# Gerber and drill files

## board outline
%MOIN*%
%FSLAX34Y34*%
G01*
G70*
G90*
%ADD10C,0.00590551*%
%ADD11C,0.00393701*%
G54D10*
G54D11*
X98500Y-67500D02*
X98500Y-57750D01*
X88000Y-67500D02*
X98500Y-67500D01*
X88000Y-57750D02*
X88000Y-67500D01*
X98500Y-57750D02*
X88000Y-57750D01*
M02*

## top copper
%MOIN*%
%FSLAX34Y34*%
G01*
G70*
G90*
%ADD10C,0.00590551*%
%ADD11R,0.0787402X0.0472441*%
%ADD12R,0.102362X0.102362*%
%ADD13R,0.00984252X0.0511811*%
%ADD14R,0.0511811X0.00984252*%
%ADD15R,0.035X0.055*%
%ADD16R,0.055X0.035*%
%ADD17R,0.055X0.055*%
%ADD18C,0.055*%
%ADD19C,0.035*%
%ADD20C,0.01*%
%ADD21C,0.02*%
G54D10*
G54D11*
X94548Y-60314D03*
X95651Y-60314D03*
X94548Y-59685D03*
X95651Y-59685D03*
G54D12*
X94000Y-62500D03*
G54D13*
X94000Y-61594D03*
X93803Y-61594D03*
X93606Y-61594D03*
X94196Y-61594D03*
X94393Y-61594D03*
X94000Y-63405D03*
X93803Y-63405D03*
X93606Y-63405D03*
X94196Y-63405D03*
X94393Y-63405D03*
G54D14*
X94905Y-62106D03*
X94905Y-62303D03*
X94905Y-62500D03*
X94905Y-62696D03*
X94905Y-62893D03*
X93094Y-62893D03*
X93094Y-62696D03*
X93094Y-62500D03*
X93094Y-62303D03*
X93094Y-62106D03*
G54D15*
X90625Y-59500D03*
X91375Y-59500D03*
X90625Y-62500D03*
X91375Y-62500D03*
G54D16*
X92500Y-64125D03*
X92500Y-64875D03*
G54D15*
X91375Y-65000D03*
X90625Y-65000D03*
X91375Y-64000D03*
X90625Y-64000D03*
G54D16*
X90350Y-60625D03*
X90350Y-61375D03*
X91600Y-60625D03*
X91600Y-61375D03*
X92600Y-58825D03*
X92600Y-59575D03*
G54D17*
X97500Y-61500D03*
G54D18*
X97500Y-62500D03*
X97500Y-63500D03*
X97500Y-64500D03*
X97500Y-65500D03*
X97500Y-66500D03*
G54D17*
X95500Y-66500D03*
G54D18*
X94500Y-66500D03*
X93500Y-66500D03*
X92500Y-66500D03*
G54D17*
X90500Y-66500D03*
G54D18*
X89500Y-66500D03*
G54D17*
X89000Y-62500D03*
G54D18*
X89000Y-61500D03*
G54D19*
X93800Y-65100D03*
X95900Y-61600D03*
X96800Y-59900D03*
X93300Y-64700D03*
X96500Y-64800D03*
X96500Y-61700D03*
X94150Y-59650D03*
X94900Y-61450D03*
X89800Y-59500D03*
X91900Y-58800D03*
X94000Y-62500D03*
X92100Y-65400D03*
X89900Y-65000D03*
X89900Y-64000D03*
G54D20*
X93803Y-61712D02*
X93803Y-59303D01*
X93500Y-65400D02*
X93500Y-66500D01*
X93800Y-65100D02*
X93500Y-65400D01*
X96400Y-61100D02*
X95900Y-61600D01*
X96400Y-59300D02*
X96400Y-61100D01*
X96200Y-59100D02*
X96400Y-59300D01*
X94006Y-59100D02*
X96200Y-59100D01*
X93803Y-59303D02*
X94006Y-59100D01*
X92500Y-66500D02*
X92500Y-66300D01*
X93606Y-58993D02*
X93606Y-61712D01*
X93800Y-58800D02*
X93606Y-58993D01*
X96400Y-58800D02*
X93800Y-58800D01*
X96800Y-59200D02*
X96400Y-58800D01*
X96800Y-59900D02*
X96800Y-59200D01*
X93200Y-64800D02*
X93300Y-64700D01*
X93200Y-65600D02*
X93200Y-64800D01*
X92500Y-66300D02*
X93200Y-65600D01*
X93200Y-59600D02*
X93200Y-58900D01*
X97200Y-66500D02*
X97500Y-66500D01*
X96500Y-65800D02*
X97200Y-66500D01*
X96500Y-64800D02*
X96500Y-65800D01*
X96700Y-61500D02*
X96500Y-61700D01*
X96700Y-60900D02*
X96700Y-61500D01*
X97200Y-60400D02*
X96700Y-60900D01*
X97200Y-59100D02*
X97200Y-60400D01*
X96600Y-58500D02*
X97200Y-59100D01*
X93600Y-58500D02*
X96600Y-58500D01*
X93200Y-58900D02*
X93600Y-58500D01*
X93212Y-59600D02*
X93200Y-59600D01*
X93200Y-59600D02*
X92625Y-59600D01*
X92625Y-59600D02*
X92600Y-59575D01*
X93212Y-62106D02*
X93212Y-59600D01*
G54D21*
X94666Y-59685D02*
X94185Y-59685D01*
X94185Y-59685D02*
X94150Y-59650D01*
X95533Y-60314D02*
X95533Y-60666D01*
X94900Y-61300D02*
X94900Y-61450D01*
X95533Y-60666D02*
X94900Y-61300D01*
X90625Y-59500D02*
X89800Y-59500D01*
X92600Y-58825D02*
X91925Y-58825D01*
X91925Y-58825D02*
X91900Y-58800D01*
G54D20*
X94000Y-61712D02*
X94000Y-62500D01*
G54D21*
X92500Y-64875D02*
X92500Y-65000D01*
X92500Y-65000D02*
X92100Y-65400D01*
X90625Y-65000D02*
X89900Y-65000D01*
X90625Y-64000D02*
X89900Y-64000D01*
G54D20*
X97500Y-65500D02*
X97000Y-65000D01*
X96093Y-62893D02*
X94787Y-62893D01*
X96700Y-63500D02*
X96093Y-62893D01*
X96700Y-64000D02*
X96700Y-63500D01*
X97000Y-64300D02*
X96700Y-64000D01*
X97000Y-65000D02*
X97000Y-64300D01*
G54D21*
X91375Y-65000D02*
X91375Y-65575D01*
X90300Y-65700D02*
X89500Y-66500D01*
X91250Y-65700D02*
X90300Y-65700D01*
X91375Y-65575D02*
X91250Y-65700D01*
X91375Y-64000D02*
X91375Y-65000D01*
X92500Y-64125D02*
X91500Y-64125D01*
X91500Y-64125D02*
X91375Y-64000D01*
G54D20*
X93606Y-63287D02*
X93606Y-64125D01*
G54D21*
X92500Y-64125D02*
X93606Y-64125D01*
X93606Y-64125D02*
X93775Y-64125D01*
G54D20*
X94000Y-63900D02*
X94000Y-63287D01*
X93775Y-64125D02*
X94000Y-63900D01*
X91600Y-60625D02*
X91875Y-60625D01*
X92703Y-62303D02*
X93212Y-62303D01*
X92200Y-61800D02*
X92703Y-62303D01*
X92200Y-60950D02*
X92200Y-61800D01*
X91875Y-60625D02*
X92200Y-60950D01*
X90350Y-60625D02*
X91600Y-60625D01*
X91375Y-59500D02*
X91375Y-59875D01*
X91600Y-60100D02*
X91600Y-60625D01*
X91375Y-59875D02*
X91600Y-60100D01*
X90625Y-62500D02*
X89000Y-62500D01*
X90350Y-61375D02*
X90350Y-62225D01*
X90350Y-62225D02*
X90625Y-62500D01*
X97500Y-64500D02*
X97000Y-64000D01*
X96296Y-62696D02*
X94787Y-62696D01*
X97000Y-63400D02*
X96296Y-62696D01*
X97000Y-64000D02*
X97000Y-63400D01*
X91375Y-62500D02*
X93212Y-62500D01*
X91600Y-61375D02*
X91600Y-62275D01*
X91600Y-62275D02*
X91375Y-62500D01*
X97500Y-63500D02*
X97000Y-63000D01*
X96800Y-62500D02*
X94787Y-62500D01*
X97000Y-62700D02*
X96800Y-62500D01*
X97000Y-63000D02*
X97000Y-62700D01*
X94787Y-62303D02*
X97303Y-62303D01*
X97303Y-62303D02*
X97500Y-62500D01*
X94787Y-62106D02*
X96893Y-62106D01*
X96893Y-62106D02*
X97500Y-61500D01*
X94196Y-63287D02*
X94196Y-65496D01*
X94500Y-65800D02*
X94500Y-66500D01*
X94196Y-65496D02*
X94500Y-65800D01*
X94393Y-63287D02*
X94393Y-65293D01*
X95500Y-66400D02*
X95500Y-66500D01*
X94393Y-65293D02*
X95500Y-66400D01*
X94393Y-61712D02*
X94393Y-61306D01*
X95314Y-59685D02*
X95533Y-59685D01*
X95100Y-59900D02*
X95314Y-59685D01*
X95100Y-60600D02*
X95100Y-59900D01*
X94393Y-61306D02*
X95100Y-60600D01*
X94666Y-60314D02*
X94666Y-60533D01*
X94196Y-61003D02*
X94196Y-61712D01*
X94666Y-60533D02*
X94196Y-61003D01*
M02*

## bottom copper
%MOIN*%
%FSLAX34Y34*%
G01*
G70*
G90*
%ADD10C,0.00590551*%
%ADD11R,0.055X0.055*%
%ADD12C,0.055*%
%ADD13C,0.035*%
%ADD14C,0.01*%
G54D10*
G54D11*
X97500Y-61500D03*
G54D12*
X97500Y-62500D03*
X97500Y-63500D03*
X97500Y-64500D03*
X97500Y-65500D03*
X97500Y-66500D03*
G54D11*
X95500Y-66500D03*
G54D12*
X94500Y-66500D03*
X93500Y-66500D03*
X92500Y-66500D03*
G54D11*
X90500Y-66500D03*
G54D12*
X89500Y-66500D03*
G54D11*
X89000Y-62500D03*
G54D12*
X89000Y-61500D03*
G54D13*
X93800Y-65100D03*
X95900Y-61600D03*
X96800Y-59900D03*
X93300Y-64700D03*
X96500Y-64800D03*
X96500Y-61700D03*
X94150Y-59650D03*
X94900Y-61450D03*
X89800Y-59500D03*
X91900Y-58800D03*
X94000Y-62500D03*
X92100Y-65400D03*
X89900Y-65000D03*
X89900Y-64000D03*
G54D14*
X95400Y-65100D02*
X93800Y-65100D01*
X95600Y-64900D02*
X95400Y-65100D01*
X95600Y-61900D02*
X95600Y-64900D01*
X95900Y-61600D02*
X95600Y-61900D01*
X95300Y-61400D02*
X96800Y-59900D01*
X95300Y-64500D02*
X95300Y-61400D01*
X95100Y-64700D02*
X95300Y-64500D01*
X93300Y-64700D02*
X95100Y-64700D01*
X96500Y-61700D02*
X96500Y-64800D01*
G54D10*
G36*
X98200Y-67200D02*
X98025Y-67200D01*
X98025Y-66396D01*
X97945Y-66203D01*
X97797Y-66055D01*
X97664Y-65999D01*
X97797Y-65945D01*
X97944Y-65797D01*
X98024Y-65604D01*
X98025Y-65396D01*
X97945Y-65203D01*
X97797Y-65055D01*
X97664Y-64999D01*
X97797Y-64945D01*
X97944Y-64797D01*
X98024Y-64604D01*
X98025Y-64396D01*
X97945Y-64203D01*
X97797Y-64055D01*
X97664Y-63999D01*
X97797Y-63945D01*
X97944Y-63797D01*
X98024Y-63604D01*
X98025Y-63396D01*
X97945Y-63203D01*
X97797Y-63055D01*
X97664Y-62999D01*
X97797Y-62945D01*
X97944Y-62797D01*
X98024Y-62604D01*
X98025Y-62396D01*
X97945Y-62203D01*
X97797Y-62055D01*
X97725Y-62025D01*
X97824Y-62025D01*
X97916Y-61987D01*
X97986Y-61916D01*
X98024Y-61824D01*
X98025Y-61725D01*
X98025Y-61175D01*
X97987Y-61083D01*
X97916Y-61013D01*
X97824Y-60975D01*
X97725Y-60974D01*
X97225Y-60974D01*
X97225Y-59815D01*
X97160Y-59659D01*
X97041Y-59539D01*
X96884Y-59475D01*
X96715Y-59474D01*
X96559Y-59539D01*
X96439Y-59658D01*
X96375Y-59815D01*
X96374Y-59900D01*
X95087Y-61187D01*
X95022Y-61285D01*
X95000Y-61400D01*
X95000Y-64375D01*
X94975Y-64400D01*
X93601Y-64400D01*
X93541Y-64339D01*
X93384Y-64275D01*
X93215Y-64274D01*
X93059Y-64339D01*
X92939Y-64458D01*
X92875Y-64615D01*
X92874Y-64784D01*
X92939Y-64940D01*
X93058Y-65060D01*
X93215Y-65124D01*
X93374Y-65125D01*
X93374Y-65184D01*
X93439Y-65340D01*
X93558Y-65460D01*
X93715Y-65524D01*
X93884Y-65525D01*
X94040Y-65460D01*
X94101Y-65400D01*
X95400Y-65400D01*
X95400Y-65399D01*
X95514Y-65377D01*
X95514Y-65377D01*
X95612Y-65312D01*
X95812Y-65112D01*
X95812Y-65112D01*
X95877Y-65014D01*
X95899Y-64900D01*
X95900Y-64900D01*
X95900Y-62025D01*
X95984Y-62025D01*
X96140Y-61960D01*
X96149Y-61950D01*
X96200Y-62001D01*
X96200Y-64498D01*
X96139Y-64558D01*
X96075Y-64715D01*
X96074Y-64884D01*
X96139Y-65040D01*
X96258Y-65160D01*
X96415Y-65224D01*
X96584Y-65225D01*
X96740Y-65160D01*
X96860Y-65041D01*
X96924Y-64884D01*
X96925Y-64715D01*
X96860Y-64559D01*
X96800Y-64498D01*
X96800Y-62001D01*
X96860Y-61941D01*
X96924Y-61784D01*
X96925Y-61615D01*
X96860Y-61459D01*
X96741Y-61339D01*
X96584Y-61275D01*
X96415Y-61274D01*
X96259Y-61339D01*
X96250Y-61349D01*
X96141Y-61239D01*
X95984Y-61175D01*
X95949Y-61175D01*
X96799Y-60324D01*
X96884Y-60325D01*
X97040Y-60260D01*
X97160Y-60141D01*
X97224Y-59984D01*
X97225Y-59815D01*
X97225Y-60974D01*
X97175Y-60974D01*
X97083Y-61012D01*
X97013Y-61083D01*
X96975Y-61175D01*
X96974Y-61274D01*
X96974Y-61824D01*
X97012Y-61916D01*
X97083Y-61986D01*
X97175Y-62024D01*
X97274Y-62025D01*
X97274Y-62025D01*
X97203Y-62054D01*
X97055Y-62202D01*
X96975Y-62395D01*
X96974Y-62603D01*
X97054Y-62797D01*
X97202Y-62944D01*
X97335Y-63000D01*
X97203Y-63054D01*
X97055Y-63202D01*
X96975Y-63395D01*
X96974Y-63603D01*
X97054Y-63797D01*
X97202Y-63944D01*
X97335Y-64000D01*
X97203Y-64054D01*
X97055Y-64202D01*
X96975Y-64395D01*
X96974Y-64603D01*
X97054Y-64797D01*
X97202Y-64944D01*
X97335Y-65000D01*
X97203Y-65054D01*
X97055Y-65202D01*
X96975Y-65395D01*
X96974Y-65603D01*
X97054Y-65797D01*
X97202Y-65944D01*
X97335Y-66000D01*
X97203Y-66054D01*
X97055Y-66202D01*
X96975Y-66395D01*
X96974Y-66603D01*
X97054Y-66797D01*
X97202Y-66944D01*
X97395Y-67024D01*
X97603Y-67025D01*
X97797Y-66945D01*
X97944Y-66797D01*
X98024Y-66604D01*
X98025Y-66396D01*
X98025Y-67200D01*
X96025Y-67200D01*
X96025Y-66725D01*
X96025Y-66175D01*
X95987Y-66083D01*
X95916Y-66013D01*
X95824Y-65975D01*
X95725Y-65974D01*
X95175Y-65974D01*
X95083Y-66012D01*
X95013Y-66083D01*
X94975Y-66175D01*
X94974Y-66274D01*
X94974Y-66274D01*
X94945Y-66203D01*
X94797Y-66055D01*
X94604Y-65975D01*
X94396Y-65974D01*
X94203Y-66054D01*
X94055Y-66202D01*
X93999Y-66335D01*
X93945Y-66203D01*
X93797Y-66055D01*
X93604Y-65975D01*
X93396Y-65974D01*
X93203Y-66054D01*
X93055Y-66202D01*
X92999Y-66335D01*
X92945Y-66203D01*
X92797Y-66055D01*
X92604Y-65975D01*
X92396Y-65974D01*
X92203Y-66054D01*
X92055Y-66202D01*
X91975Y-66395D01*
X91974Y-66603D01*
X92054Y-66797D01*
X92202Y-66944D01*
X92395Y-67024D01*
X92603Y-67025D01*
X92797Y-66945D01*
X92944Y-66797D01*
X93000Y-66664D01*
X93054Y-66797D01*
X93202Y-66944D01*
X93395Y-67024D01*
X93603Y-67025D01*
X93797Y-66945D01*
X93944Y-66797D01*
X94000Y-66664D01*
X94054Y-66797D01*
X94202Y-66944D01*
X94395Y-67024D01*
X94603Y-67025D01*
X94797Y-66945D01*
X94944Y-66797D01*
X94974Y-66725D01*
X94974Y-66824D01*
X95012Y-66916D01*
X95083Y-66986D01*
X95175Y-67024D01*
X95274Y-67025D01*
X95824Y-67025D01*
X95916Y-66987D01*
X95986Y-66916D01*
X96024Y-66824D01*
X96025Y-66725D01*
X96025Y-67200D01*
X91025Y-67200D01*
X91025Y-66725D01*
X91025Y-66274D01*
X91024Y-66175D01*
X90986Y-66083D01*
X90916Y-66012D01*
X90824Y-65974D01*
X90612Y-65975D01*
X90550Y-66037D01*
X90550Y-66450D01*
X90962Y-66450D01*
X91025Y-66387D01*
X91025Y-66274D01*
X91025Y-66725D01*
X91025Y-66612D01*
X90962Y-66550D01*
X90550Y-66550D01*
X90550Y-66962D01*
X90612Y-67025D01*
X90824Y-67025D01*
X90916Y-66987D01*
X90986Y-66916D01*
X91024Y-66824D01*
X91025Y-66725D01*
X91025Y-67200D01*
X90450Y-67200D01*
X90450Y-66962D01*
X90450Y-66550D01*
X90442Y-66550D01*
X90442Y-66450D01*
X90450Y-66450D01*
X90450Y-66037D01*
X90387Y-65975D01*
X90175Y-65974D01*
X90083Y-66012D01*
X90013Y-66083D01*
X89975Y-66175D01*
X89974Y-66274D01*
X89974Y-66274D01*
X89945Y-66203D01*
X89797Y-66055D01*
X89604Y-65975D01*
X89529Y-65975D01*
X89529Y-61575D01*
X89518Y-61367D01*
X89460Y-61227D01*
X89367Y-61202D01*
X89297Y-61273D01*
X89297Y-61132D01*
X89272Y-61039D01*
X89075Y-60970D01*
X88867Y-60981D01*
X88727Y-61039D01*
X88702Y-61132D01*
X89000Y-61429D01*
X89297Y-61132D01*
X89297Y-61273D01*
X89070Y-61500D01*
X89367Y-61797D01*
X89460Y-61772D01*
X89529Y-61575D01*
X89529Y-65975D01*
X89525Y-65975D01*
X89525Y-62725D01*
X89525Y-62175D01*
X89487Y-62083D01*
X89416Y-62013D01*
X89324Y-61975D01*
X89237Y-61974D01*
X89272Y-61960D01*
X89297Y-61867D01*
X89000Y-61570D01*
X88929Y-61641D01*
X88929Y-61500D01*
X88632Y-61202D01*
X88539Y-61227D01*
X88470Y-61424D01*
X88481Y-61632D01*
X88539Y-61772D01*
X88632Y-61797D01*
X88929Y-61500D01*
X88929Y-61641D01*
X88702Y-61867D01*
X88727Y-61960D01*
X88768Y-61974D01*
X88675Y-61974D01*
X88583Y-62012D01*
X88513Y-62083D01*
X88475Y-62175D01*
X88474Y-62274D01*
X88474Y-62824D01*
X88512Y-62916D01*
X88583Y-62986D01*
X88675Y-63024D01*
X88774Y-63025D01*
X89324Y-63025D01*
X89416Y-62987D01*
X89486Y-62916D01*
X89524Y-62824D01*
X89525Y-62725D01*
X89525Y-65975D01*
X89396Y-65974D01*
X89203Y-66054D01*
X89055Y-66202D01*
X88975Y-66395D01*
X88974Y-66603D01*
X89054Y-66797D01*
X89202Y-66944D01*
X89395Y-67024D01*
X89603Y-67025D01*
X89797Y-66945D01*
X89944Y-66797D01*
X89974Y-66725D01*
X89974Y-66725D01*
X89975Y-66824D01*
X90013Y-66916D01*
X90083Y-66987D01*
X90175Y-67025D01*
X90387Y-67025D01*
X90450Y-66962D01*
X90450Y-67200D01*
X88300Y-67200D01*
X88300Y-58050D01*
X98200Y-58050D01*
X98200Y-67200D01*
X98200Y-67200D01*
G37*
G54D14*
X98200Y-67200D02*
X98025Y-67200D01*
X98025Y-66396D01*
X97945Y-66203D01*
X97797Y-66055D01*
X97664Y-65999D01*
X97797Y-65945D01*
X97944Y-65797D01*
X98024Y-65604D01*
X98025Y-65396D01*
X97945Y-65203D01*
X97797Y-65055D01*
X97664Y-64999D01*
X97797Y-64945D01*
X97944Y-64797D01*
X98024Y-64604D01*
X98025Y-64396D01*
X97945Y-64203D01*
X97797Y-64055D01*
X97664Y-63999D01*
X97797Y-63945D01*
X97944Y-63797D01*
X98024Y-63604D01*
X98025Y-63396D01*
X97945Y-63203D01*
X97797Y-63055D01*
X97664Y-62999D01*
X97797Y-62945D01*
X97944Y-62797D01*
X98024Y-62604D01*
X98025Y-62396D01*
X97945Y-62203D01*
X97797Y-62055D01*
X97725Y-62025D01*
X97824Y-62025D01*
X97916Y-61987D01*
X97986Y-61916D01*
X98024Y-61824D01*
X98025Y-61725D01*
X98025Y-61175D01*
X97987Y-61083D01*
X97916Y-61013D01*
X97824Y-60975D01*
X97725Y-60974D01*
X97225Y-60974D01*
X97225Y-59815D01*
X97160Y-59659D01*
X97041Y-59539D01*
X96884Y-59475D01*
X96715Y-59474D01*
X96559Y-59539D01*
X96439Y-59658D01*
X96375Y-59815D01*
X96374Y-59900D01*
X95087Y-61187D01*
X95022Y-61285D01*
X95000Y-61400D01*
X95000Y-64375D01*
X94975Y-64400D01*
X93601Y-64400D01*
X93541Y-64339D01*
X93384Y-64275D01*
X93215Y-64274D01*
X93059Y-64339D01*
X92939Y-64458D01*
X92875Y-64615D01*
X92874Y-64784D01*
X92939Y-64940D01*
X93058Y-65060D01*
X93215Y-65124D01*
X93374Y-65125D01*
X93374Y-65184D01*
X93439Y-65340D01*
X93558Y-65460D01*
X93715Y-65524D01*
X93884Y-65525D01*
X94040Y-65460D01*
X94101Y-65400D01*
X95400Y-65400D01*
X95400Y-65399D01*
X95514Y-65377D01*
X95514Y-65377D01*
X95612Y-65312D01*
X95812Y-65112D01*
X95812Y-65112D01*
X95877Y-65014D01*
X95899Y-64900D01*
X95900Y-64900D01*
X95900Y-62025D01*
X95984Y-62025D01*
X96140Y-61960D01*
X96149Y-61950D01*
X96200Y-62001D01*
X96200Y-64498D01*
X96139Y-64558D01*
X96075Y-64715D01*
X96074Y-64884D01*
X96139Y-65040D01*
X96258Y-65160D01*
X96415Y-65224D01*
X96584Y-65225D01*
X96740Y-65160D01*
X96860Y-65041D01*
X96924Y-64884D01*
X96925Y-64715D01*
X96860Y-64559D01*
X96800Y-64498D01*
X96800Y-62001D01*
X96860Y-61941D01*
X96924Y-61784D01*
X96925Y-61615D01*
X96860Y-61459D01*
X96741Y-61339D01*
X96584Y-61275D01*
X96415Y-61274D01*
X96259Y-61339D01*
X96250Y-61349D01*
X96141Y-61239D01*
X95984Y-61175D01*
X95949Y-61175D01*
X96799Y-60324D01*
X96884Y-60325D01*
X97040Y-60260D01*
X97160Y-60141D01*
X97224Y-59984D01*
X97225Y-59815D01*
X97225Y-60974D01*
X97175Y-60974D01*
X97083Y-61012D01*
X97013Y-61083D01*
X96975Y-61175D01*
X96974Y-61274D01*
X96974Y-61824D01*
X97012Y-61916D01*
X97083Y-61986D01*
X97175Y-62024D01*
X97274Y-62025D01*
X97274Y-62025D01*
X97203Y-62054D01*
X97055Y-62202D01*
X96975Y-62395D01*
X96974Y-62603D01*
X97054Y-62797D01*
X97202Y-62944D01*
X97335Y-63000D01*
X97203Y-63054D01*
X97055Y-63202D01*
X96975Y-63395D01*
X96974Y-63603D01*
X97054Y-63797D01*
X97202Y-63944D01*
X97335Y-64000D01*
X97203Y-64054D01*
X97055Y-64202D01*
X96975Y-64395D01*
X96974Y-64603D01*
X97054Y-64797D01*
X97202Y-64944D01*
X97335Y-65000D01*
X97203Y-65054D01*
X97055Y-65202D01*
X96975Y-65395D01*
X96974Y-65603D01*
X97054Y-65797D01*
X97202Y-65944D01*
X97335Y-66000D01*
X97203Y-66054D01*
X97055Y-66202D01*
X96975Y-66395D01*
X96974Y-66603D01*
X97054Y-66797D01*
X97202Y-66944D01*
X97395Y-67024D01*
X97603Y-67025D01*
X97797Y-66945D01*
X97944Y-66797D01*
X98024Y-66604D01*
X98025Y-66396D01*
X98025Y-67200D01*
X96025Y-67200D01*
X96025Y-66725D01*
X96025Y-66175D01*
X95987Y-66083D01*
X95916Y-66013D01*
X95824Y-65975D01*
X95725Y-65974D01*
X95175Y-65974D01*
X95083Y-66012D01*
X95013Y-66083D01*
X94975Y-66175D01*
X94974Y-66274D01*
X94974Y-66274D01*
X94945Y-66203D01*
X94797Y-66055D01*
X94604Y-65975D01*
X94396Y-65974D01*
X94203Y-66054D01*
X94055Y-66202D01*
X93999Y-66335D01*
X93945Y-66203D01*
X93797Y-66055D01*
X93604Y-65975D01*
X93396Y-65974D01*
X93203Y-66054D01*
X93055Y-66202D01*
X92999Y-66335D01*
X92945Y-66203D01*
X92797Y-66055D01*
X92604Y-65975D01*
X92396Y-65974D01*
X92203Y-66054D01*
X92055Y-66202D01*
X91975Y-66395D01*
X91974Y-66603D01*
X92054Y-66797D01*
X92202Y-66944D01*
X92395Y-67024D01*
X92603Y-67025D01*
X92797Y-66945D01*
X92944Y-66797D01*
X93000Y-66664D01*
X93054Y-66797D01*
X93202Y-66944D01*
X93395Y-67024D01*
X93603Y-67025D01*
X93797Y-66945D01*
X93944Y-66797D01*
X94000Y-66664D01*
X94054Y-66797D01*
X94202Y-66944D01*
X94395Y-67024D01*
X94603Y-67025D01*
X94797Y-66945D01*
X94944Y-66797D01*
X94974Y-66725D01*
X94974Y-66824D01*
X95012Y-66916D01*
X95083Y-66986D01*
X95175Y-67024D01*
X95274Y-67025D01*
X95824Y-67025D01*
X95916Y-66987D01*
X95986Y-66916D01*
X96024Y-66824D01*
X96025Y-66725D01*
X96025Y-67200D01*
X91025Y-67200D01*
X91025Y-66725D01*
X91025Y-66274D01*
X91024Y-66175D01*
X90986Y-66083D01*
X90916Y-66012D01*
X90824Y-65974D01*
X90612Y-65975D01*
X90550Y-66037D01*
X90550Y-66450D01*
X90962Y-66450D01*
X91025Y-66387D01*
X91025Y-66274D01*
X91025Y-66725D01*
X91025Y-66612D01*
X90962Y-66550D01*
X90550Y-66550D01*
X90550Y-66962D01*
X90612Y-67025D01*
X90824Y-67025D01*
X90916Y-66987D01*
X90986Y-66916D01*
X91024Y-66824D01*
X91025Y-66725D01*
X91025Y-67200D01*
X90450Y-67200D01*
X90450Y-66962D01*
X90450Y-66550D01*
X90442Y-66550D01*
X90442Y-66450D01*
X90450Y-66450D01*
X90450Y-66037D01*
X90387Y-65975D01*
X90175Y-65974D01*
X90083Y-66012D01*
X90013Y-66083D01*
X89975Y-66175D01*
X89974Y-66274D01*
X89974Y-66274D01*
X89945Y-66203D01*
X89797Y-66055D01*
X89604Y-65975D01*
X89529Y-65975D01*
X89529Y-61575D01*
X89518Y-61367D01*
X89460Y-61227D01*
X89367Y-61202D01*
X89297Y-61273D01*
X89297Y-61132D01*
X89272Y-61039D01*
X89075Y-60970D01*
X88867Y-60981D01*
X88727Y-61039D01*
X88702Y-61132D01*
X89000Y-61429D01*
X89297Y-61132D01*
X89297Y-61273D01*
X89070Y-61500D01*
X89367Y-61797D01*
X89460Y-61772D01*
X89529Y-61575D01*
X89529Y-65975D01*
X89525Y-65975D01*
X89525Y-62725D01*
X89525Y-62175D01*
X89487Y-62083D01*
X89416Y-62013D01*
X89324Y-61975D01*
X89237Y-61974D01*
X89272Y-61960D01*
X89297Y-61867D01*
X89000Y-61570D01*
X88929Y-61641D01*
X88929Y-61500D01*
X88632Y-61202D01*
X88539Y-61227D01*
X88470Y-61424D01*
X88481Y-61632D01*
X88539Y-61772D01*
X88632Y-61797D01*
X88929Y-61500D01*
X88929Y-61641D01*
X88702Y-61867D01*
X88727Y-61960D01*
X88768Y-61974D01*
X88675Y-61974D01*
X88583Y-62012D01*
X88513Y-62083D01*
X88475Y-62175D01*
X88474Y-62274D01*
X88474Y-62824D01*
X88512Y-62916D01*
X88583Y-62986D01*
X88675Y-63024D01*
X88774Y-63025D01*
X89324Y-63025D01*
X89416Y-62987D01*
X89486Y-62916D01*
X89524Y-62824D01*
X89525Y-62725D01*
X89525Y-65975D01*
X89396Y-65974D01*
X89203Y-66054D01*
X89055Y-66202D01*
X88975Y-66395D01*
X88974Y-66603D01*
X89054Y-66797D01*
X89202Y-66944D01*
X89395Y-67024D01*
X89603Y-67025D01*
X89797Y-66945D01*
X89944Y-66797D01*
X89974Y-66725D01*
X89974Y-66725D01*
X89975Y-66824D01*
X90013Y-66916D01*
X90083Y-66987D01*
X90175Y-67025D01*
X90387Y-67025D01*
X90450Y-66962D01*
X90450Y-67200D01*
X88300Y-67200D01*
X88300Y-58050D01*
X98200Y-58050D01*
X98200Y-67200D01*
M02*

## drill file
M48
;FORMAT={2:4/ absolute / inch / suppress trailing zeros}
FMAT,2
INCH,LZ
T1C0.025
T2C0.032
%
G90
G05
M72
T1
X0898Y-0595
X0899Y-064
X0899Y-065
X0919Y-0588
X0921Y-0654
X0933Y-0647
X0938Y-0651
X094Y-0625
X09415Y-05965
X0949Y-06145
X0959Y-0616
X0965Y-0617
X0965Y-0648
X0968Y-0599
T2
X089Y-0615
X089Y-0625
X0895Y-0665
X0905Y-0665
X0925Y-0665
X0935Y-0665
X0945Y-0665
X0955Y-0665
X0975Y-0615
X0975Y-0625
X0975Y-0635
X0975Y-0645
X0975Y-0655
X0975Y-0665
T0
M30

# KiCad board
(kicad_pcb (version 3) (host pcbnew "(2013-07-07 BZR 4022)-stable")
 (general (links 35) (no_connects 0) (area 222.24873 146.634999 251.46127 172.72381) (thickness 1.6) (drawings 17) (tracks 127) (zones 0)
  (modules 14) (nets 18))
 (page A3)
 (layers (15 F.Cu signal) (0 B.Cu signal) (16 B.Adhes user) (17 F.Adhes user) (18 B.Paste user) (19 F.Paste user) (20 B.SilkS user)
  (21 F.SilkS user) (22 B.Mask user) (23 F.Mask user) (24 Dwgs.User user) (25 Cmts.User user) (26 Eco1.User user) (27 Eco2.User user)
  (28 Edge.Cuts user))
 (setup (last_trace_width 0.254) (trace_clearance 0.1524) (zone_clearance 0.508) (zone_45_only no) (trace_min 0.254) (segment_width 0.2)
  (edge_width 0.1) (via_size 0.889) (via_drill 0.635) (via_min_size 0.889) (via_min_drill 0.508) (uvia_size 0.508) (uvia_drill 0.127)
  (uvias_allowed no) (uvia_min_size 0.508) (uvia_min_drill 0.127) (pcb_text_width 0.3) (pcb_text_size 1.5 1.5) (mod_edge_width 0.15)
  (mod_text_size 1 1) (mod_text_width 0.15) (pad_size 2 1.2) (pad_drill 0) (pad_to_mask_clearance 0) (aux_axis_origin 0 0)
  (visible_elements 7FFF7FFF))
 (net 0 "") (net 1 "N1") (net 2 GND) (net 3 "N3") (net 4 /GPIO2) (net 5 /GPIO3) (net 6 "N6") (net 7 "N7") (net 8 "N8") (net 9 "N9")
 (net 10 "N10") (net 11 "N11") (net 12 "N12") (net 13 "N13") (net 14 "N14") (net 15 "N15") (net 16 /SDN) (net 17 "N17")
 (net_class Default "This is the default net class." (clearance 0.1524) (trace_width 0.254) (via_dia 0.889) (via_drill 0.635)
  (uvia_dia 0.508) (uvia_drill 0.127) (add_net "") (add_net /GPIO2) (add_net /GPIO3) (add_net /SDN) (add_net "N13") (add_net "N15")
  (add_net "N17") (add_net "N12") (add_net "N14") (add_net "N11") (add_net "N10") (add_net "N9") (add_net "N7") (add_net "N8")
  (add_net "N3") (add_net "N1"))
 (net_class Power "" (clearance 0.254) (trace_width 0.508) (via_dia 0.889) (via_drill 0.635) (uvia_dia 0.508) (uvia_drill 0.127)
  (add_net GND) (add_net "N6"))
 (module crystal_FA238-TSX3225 (layer F.Cu) (at 241.554 152.4)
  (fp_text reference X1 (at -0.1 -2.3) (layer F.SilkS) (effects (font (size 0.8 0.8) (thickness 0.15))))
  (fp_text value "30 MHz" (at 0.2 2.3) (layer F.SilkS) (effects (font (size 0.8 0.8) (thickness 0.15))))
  (pad 1 smd rect (at -1.4 0.8) (size 2 1.2) (layers F.Cu F.Paste F.Mask) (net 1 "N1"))
  (pad 3 smd rect (at 1.1 0.8) (size 2 1.2) (drill (offset 0.3 0)) (layers F.Cu F.Paste F.Mask) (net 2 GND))
  (pad 3 smd rect (at -1.4 -0.8) (size 2 1.2) (layers F.Cu F.Paste F.Mask) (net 2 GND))
  (pad 2 smd rect (at 1.1 -0.8) (size 2 1.2) (drill (offset 0.3 0)) (layers F.Cu F.Paste F.Mask) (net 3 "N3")))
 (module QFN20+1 (layer F.Cu) (at 238.76 158.75)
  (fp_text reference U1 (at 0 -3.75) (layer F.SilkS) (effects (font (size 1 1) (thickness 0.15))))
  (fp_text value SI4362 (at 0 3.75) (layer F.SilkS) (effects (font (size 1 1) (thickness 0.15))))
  (pad 21 smd rect (at 0 0) (size 2.6 2.6) (layers F.Cu F.Paste F.Mask) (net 2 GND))
  (pad 18 smd rect (at 0 -2.3) (size 0.25 1.3) (layers F.Cu F.Paste F.Mask) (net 2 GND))
  (pad 19 smd rect (at -0.5 -2.3) (size 0.25 1.3) (layers F.Cu F.Paste F.Mask) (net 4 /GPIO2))
  (pad 20 smd rect (at -1 -2.3) (size 0.25 1.3) (layers F.Cu F.Paste F.Mask) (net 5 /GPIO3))
  (pad 17 smd rect (at 0.5 -2.3) (size 0.25 1.3) (layers F.Cu F.Paste F.Mask) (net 1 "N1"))
  (pad 16 smd rect (at 1 -2.3) (size 0.25 1.3) (layers F.Cu F.Paste F.Mask) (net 3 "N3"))
  (pad 8 smd rect (at 0 2) (size 0.25 1.3) (drill (offset 0 0.3)) (layers F.Cu F.Paste F.Mask) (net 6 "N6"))
  (pad 7 smd rect (at -0.5 2) (size 0.25 1.3) (drill (offset 0 0.3)) (layers F.Cu F.Paste F.Mask))
  (pad 6 smd rect (at -1 2) (size 0.25 1.3) (drill (offset 0 0.3)) (layers F.Cu F.Paste F.Mask) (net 6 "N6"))
  (pad 9 smd rect (at 0.5 2) (size 0.25 1.3) (drill (offset 0 0.3)) (layers F.Cu F.Paste F.Mask) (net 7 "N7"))
  (pad 10 smd rect (at 1 2) (size 0.25 1.3) (drill (offset 0 0.3)) (layers F.Cu F.Paste F.Mask) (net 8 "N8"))
  (pad 15 smd rect (at 2 -1) (size 1.3 0.25) (drill (offset 0.3 0)) (layers F.Cu F.Paste F.Mask) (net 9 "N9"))
  (pad 14 smd rect (at 2 -0.5) (size 1.3 0.25) (drill (offset 0.3 0)) (layers F.Cu F.Paste F.Mask) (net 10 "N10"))
  (pad 13 smd rect (at 2 0) (size 1.3 0.25) (drill (offset 0.3 0)) (layers F.Cu F.Paste F.Mask) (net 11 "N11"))
  (pad 12 smd rect (at 2 0.5) (size 1.3 0.25) (drill (offset 0.3 0)) (layers F.Cu F.Paste F.Mask) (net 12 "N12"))
  (pad 11 smd rect (at 2 1) (size 1.3 0.25) (drill (offset 0.3 0)) (layers F.Cu F.Paste F.Mask) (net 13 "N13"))
  (pad 5 smd rect (at -2.3 1) (size 1.3 0.25) (layers F.Cu F.Paste F.Mask))
  (pad 4 smd rect (at -2.3 0.5) (size 1.3 0.25) (layers F.Cu F.Paste F.Mask))
  (pad 3 smd rect (at -2.3 0) (size 1.3 0.25) (layers F.Cu F.Paste F.Mask) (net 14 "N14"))
  (pad 2 smd rect (at -2.3 -0.5) (size 1.3 0.25) (layers F.Cu F.Paste F.Mask) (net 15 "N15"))
  (pad 1 smd rect (at -2.3 -1) (size 1.3 0.25) (layers F.Cu F.Paste F.Mask) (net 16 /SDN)))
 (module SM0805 (layer F.Cu) (at 231.14 151.13)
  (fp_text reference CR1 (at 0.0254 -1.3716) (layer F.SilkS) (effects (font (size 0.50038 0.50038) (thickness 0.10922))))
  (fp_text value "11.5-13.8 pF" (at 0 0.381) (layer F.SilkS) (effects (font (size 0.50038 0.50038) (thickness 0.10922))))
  (pad 1 smd rect (at -0.9525 0) (size 0.889 1.397) (layers F.Cu F.Paste F.Mask) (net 2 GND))
  (pad 2 smd rect (at 0.9525 0) (size 0.889 1.397) (layers F.Cu F.Paste F.Mask) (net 15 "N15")))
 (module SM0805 (layer F.Cu) (at 231.14 158.75)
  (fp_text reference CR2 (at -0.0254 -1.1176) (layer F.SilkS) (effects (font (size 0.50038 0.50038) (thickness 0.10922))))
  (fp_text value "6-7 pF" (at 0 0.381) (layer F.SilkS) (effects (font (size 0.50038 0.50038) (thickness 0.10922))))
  (pad 1 smd rect (at -0.9525 0) (size 0.889 1.397) (layers F.Cu F.Paste F.Mask) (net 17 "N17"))
  (pad 2 smd rect (at 0.9525 0) (size 0.889 1.397) (layers F.Cu F.Paste F.Mask) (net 14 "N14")))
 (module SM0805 (layer F.Cu) (at 234.95 163.83 270)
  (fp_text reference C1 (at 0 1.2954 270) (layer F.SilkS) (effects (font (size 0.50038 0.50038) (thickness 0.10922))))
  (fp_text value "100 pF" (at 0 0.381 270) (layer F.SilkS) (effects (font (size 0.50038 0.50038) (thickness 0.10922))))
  (pad 1 smd rect (at -0.9525 0 270) (size 0.889 1.397) (layers F.Cu F.Paste F.Mask) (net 6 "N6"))
  (pad 2 smd rect (at 0.9525 0 270) (size 0.889 1.397) (layers F.Cu F.Paste F.Mask) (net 2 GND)))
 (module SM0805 (layer F.Cu) (at 231.14 165.1 180)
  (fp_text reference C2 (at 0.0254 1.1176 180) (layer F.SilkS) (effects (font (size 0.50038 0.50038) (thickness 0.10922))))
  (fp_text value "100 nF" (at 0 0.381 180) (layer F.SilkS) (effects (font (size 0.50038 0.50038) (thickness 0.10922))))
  (pad 1 smd rect (at -0.9525 0 180) (size 0.889 1.397) (layers F.Cu F.Paste F.Mask) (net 6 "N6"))
  (pad 2 smd rect (at 0.9525 0 180) (size 0.889 1.397) (layers F.Cu F.Paste F.Mask) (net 2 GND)))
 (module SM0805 (layer F.Cu) (at 231.14 162.56 180)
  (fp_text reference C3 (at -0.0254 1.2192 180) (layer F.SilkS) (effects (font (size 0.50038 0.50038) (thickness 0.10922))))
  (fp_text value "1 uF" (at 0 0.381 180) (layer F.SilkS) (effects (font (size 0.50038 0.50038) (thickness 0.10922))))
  (pad 1 smd rect (at -0.9525 0 180) (size 0.889 1.397) (layers F.Cu F.Paste F.Mask) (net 6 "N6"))
  (pad 2 smd rect (at 0.9525 0 180) (size 0.889 1.397) (layers F.Cu F.Paste F.Mask) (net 2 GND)))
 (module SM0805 (layer F.Cu) (at 229.489 154.94 270)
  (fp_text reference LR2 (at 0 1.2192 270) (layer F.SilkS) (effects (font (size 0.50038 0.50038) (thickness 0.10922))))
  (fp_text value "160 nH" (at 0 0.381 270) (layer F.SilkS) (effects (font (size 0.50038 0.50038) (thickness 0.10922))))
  (pad 1 smd rect (at -0.9525 0 270) (size 0.889 1.397) (layers F.Cu F.Paste F.Mask) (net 15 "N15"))
  (pad 2 smd rect (at 0.9525 0 270) (size 0.889 1.397) (layers F.Cu F.Paste F.Mask) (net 17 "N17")))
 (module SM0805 (layer F.Cu) (at 232.664 154.94 270)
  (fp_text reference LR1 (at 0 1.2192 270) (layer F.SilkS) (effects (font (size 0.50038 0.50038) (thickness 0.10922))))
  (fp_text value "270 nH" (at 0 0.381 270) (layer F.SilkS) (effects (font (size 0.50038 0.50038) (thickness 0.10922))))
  (pad 1 smd rect (at -0.9525 0 270) (size 0.889 1.397) (layers F.Cu F.Paste F.Mask) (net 15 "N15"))
  (pad 2 smd rect (at 0.9525 0 270) (size 0.889 1.397) (layers F.Cu F.Paste F.Mask) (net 14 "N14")))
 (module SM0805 (layer F.Cu) (at 235.204 150.368 270)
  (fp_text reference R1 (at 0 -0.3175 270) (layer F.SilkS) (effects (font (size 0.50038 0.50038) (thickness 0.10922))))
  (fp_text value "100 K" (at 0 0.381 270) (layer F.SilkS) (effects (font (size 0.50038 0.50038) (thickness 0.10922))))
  (pad 1 smd rect (at -0.9525 0 270) (size 0.889 1.397) (layers F.Cu F.Paste F.Mask) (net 2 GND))
  (pad 2 smd rect (at 0.9525 0 270) (size 0.889 1.397) (layers F.Cu F.Paste F.Mask) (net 16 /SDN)))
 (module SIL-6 (layer F.Cu) (at 247.65 162.56 270)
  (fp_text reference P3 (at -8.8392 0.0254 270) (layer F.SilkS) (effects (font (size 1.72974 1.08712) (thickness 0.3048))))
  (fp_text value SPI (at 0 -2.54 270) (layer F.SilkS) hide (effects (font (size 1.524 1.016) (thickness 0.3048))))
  (pad 1 thru_hole rect (at -6.35 0 270) (size 1.397 1.397) (drill 0.8128) (layers *.Cu *.Mask F.SilkS) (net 9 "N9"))
  (pad 2 thru_hole circle (at -3.81 0 270) (size 1.397 1.397) (drill 0.8128) (layers *.Cu *.Mask F.SilkS) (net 10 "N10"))
  (pad 3 thru_hole circle (at -1.27 0 270) (size 1.397 1.397) (drill 0.8128) (layers *.Cu *.Mask F.SilkS) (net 11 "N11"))
  (pad 4 thru_hole circle (at 1.27 0 270) (size 1.397 1.397) (drill 0.8128) (layers *.Cu *.Mask F.SilkS) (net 12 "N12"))
  (pad 5 thru_hole circle (at 3.81 0 270) (size 1.397 1.397) (drill 0.8128) (layers *.Cu *.Mask F.SilkS) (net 13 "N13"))
  (pad 6 thru_hole circle (at 6.35 0 270) (size 1.397 1.397) (drill 0.8128) (layers *.Cu *.Mask F.SilkS) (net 16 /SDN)))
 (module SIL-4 (layer F.Cu) (at 238.76 168.91 180)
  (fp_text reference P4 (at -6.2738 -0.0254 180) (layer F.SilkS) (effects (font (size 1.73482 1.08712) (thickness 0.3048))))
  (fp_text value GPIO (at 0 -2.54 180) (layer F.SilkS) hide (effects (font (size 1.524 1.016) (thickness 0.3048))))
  (pad 1 thru_hole rect (at -3.81 0 180) (size 1.397 1.397) (drill 0.8128) (layers *.Cu *.Mask F.SilkS) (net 8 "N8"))
  (pad 2 thru_hole circle (at -1.27 0 180) (size 1.397 1.397) (drill 0.8128) (layers *.Cu *.Mask F.SilkS) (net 7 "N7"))
  (pad 3 thru_hole circle (at 1.27 0 180) (size 1.397 1.397) (drill 0.8128) (layers *.Cu *.Mask F.SilkS) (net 4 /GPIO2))
  (pad 4 thru_hole circle (at 3.81 0 180) (size 1.397 1.397) (drill 0.8128) (layers *.Cu *.Mask F.SilkS) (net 5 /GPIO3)))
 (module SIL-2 (layer F.Cu) (at 228.6 168.91 180)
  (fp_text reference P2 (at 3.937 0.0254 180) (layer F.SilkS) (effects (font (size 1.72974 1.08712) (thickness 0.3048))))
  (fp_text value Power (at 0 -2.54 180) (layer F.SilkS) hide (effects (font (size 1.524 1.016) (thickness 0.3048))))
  (pad 1 thru_hole rect (at -1.27 0 180) (size 1.397 1.397) (drill 0.8128) (layers *.Cu *.Mask F.SilkS) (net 2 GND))
  (pad 2 thru_hole circle (at 1.27 0 180) (size 1.397 1.397) (drill 0.8128) (layers *.Cu *.Mask F.SilkS) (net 6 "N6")))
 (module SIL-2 (layer F.Cu) (at 226.06 157.48 90)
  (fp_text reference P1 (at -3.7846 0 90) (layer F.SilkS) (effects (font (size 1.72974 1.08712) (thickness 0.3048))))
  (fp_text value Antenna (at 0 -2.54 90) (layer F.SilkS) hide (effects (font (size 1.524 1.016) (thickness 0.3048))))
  (pad 1 thru_hole rect (at -1.27 0 90) (size 1.397 1.397) (drill 0.8128) (layers *.Cu *.Mask F.SilkS) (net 17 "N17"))
  (pad 2 thru_hole circle (at 1.27 0 90) (size 1.397 1.397) (drill 0.8128) (layers *.Cu *.Mask F.SilkS) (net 2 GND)))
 (gr_line (start 250.19 171.45) (end 250.19 146.685) (angle 90) (layer Edge.Cuts) (width 0.1))
 (gr_line (start 223.52 171.45) (end 250.19 171.45) (angle 90) (layer Edge.Cuts) (width 0.1))
 (gr_line (start 223.52 146.685) (end 223.52 171.45) (angle 90) (layer Edge.Cuts) (width 0.1))
 (gr_line (start 250.19 146.685) (end 223.52 146.685) (angle 90) (layer Edge.Cuts) (width 0.1))
 (segment (start 238.26 156.75) (end 238.26 150.63) (width 0.254) (layer F.Cu) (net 4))
 (segment (start 237.49 166.116) (end 237.49 168.91) (width 0.254) (layer F.Cu) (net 4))
 (segment (start 238.252 165.354) (end 237.49 166.116) (width 0.254) (layer F.Cu) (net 4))
 (via (at 238.252 165.354) (size 0.889) (layers F.Cu B.Cu) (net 4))
 (segment (start 242.316 165.354) (end 238.252 165.354) (width 0.254) (layer B.Cu) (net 4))
 (segment (start 242.824 164.846) (end 242.316 165.354) (width 0.254) (layer B.Cu) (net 4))
 (segment (start 242.824 157.226) (end 242.824 164.846) (width 0.254) (layer B.Cu) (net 4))
 (segment (start 243.586 156.464) (end 242.824 157.226) (width 0.254) (layer B.Cu) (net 4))
 (via (at 243.586 156.464) (size 0.889) (layers F.Cu B.Cu) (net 4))
 (segment (start 244.856 155.194) (end 243.586 156.464) (width 0.254) (layer F.Cu) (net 4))
 (segment (start 244.856 150.622) (end 244.856 155.194) (width 0.254) (layer F.Cu) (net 4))
 (segment (start 244.348 150.114) (end 244.856 150.622) (width 0.254) (layer F.Cu) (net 4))
 (segment (start 238.776 150.114) (end 244.348 150.114) (width 0.254) (layer F.Cu) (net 4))
 (segment (start 238.26 150.63) (end 238.776 150.114) (width 0.254) (layer F.Cu) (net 4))
 (segment (start 234.95 168.91) (end 234.95 168.402) (width 0.254) (layer F.Cu) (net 5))
 (segment (start 237.76 149.844) (end 237.76 156.75) (width 0.254) (layer F.Cu) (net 5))
 (segment (start 238.252 149.352) (end 237.76 149.844) (width 0.254) (layer F.Cu) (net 5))
 (segment (start 244.856 149.352) (end 238.252 149.352) (width 0.254) (layer F.Cu) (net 5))
 (segment (start 245.872 150.368) (end 244.856 149.352) (width 0.254) (layer F.Cu) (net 5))
 (segment (start 245.872 152.146) (end 245.872 150.368) (width 0.254) (layer F.Cu) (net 5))
 (via (at 245.872 152.146) (size 0.889) (layers F.Cu B.Cu) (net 5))
 (segment (start 242.062 155.956) (end 245.872 152.146) (width 0.254) (layer B.Cu) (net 5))
 (segment (start 242.062 163.83) (end 242.062 155.956) (width 0.254) (layer B.Cu) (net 5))
 (segment (start 241.554 164.338) (end 242.062 163.83) (width 0.254) (layer B.Cu) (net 5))
 (segment (start 236.982 164.338) (end 241.554 164.338) (width 0.254) (layer B.Cu) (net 5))
 (via (at 236.982 164.338) (size 0.889) (layers F.Cu B.Cu) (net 5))
 (segment (start 236.728 164.592) (end 236.982 164.338) (width 0.254) (layer F.Cu) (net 5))
 (segment (start 236.728 166.624) (end 236.728 164.592) (width 0.254) (layer F.Cu) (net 5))
 (segment (start 234.95 168.402) (end 236.728 166.624) (width 0.254) (layer F.Cu) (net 5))
 (segment (start 236.728 151.384) (end 236.728 149.606) (width 0.254) (layer F.Cu) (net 16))
 (segment (start 246.888 168.91) (end 247.65 168.91) (width 0.254) (layer F.Cu) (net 16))
 (segment (start 245.11 167.132) (end 246.888 168.91) (width 0.254) (layer F.Cu) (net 16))
 (segment (start 245.11 164.592) (end 245.11 167.132) (width 0.254) (layer F.Cu) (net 16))
 (via (at 245.11 164.592) (size 0.889) (layers F.Cu B.Cu) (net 16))
 (segment (start 245.11 156.718) (end 245.11 164.592) (width 0.254) (layer B.Cu) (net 16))
 (via (at 245.11 156.718) (size 0.889) (layers F.Cu B.Cu) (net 16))
 (segment (start 245.618 156.21) (end 245.11 156.718) (width 0.254) (layer F.Cu) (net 16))
 (segment (start 245.618 154.686) (end 245.618 156.21) (width 0.254) (layer F.Cu) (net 16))
 (segment (start 246.888 153.416) (end 245.618 154.686) (width 0.254) (layer F.Cu) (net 16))
 (segment (start 246.888 150.114) (end 246.888 153.416) (width 0.254) (layer F.Cu) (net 16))
 (segment (start 245.364 148.59) (end 246.888 150.114) (width 0.254) (layer F.Cu) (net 16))
 (segment (start 237.744 148.59) (end 245.364 148.59) (width 0.254) (layer F.Cu) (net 16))
 (segment (start 236.728 149.606) (end 237.744 148.59) (width 0.254) (layer F.Cu) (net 16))
 (segment (start 236.76 151.384) (end 236.728 151.384) (width 0.254) (layer F.Cu) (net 16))
 (segment (start 236.728 151.384) (end 235.2675 151.384) (width 0.254) (layer F.Cu) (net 16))
 (segment (start 235.2675 151.384) (end 235.204 151.3205) (width 0.254) (layer F.Cu) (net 16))
 (segment (start 236.76 157.75) (end 236.76 151.384) (width 0.254) (layer F.Cu) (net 16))
 (segment (start 240.454 151.6) (end 239.23 151.6) (width 0.508) (layer F.Cu) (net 2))
 (via (at 239.141 151.511) (size 0.889) (layers F.Cu B.Cu) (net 2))
 (segment (start 239.23 151.6) (end 239.141 151.511) (width 0.508) (layer F.Cu) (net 2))
 (segment (start 242.654 153.2) (end 242.654 154.094) (width 0.508) (layer F.Cu) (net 2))
 (via (at 241.046 156.083) (size 0.889) (layers F.Cu B.Cu) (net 2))
 (segment (start 241.046 155.702) (end 241.046 156.083) (width 0.508) (layer F.Cu) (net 2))
 (segment (start 242.654 154.094) (end 241.046 155.702) (width 0.508) (layer F.Cu) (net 2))
 (segment (start 230.1875 151.13) (end 228.092 151.13) (width 0.508) (layer F.Cu) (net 2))
 (via (at 228.092 151.13) (size 0.889) (layers F.Cu B.Cu) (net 2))
 (segment (start 235.204 149.4155) (end 233.4895 149.4155) (width 0.508) (layer F.Cu) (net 2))
 (segment (start 233.4895 149.4155) (end 233.426 149.352) (width 0.508) (layer F.Cu) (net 2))
 (via (at 233.426 149.352) (size 0.889) (layers F.Cu B.Cu) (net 2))
 (segment (start 238.76 156.75) (end 238.76 158.75) (width 0.254) (layer F.Cu) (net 2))
 (via (at 238.76 158.75) (size 0.889) (layers F.Cu B.Cu) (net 2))
 (via (at 233.934 166.116) (size 0.889) (layers F.Cu B.Cu) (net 2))
 (segment (start 234.95 164.7825) (end 234.95 165.1) (width 0.508) (layer F.Cu) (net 2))
 (segment (start 234.95 165.1) (end 233.934 166.116) (width 0.508) (layer F.Cu) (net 2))
 (segment (start 230.1875 165.1) (end 228.346 165.1) (width 0.508) (layer F.Cu) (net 2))
 (via (at 228.346 165.1) (size 0.889) (layers F.Cu B.Cu) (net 2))
 (segment (start 230.1875 162.56) (end 228.346 162.56) (width 0.508) (layer F.Cu) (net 2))
 (via (at 228.346 162.56) (size 0.889) (layers F.Cu B.Cu) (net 2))
 (segment (start 247.65 166.37) (end 246.38 165.1) (width 0.254) (layer F.Cu) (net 13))
 (segment (start 244.078 159.75) (end 240.76 159.75) (width 0.254) (layer F.Cu) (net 13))
 (segment (start 245.618 161.29) (end 244.078 159.75) (width 0.254) (layer F.Cu) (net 13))
 (segment (start 245.618 162.56) (end 245.618 161.29) (width 0.254) (layer F.Cu) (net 13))
 (segment (start 246.38 163.322) (end 245.618 162.56) (width 0.254) (layer F.Cu) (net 13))
 (segment (start 246.38 165.1) (end 246.38 163.322) (width 0.254) (layer F.Cu) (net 13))
 (segment (start 232.0925 165.1) (end 232.0925 166.5605) (width 0.508) (layer F.Cu) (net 6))
 (segment (start 229.362 166.878) (end 227.33 168.91) (width 0.508) (layer F.Cu) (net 6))
 (segment (start 231.775 166.878) (end 229.362 166.878) (width 0.508) (layer F.Cu) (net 6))
 (segment (start 232.0925 166.5605) (end 231.775 166.878) (width 0.508) (layer F.Cu) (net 6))
 (segment (start 232.0925 162.56) (end 232.0925 165.1) (width 0.508) (layer F.Cu) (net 6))
 (segment (start 234.95 162.8775) (end 232.41 162.8775) (width 0.508) (layer F.Cu) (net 6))
 (segment (start 232.41 162.8775) (end 232.0925 162.56) (width 0.508) (layer F.Cu) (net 6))
 (segment (start 237.76 160.75) (end 237.76 162.8775) (width 0.254) (layer F.Cu) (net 6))
 (segment (start 234.95 162.8775) (end 237.76 162.8775) (width 0.508) (layer F.Cu) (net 6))
 (segment (start 237.76 162.8775) (end 238.1885 162.8775) (width 0.508) (layer F.Cu) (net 6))
 (segment (start 238.76 162.306) (end 238.76 160.75) (width 0.254) (layer F.Cu) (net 6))
 (segment (start 238.1885 162.8775) (end 238.76 162.306) (width 0.254) (layer F.Cu) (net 6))
 (segment (start 232.664 153.9875) (end 233.3625 153.9875) (width 0.254) (layer F.Cu) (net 15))
 (segment (start 235.466 158.25) (end 236.76 158.25) (width 0.254) (layer F.Cu) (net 15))
 (segment (start 234.188 156.972) (end 235.466 158.25) (width 0.254) (layer F.Cu) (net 15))
 (segment (start 234.188 154.813) (end 234.188 156.972) (width 0.254) (layer F.Cu) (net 15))
 (segment (start 233.3625 153.9875) (end 234.188 154.813) (width 0.254) (layer F.Cu) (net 15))
 (segment (start 229.489 153.9875) (end 232.664 153.9875) (width 0.254) (layer F.Cu) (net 15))
 (segment (start 232.0925 151.13) (end 232.0925 152.0825) (width 0.254) (layer F.Cu) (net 15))
 (segment (start 232.664 152.654) (end 232.664 153.9875) (width 0.254) (layer F.Cu) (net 15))
 (segment (start 232.0925 152.0825) (end 232.664 152.654) (width 0.254) (layer F.Cu) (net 15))
 (segment (start 230.1875 158.75) (end 226.06 158.75) (width 0.254) (layer F.Cu) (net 17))
 (segment (start 229.489 155.8925) (end 229.489 158.0515) (width 0.254) (layer F.Cu) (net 17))
 (segment (start 229.489 158.0515) (end 230.1875 158.75) (width 0.254) (layer F.Cu) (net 17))
 (segment (start 247.65 163.83) (end 246.38 162.56) (width 0.254) (layer F.Cu) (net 12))
 (segment (start 244.594 159.25) (end 240.76 159.25) (width 0.254) (layer F.Cu) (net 12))
 (segment (start 246.38 161.036) (end 244.594 159.25) (width 0.254) (layer F.Cu) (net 12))
 (segment (start 246.38 162.56) (end 246.38 161.036) (width 0.254) (layer F.Cu) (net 12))
 (segment (start 232.0925 158.75) (end 236.76 158.75) (width 0.254) (layer F.Cu) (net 14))
 (segment (start 232.664 155.8925) (end 232.664 158.1785) (width 0.254) (layer F.Cu) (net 14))
 (segment (start 232.664 158.1785) (end 232.0925 158.75) (width 0.254) (layer F.Cu) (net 14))
 (segment (start 247.65 161.29) (end 246.38 160.02) (width 0.254) (layer F.Cu) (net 11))
 (segment (start 245.872 158.75) (end 240.76 158.75) (width 0.254) (layer F.Cu) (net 11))
 (segment (start 246.38 159.258) (end 245.872 158.75) (width 0.254) (layer F.Cu) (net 11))
 (segment (start 246.38 160.02) (end 246.38 159.258) (width 0.254) (layer F.Cu) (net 11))
 (segment (start 240.76 158.25) (end 247.15 158.25) (width 0.254) (layer F.Cu) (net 10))
 (segment (start 247.15 158.25) (end 247.65 158.75) (width 0.254) (layer F.Cu) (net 10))
 (segment (start 240.76 157.75) (end 246.11 157.75) (width 0.254) (layer F.Cu) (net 9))
 (segment (start 246.11 157.75) (end 247.65 156.21) (width 0.254) (layer F.Cu) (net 9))
 (segment (start 239.26 160.75) (end 239.26 166.362) (width 0.254) (layer F.Cu) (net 7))
 (segment (start 240.03 167.132) (end 240.03 168.91) (width 0.254) (layer F.Cu) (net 7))
 (segment (start 239.26 166.362) (end 240.03 167.132) (width 0.254) (layer F.Cu) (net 7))
 (segment (start 239.76 160.75) (end 239.76 165.846) (width 0.254) (layer F.Cu) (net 8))
 (segment (start 242.57 168.656) (end 242.57 168.91) (width 0.254) (layer F.Cu) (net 8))
 (segment (start 239.76 165.846) (end 242.57 168.656) (width 0.254) (layer F.Cu) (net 8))
 (segment (start 239.76 156.75) (end 239.76 155.718) (width 0.254) (layer F.Cu) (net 3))
 (segment (start 242.1 151.6) (end 242.654 151.6) (width 0.254) (layer F.Cu) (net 3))
 (segment (start 241.554 152.146) (end 242.1 151.6) (width 0.254) (layer F.Cu) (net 3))
 (segment (start 241.554 153.924) (end 241.554 152.146) (width 0.254) (layer F.Cu) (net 3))
 (segment (start 239.76 155.718) (end 241.554 153.924) (width 0.254) (layer F.Cu) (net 3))
 (segment (start 240.454 153.2) (end 240.454 153.754) (width 0.254) (layer F.Cu) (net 1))
 (segment (start 239.26 154.948) (end 239.26 156.75) (width 0.254) (layer F.Cu) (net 1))
 (segment (start 240.454 153.754) (end 239.26 154.948) (width 0.254) (layer F.Cu) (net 1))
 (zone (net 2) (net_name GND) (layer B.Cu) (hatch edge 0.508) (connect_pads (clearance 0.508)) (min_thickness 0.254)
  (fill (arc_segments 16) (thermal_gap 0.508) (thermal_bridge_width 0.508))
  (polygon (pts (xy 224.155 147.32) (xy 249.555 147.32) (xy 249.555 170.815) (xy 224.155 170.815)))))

